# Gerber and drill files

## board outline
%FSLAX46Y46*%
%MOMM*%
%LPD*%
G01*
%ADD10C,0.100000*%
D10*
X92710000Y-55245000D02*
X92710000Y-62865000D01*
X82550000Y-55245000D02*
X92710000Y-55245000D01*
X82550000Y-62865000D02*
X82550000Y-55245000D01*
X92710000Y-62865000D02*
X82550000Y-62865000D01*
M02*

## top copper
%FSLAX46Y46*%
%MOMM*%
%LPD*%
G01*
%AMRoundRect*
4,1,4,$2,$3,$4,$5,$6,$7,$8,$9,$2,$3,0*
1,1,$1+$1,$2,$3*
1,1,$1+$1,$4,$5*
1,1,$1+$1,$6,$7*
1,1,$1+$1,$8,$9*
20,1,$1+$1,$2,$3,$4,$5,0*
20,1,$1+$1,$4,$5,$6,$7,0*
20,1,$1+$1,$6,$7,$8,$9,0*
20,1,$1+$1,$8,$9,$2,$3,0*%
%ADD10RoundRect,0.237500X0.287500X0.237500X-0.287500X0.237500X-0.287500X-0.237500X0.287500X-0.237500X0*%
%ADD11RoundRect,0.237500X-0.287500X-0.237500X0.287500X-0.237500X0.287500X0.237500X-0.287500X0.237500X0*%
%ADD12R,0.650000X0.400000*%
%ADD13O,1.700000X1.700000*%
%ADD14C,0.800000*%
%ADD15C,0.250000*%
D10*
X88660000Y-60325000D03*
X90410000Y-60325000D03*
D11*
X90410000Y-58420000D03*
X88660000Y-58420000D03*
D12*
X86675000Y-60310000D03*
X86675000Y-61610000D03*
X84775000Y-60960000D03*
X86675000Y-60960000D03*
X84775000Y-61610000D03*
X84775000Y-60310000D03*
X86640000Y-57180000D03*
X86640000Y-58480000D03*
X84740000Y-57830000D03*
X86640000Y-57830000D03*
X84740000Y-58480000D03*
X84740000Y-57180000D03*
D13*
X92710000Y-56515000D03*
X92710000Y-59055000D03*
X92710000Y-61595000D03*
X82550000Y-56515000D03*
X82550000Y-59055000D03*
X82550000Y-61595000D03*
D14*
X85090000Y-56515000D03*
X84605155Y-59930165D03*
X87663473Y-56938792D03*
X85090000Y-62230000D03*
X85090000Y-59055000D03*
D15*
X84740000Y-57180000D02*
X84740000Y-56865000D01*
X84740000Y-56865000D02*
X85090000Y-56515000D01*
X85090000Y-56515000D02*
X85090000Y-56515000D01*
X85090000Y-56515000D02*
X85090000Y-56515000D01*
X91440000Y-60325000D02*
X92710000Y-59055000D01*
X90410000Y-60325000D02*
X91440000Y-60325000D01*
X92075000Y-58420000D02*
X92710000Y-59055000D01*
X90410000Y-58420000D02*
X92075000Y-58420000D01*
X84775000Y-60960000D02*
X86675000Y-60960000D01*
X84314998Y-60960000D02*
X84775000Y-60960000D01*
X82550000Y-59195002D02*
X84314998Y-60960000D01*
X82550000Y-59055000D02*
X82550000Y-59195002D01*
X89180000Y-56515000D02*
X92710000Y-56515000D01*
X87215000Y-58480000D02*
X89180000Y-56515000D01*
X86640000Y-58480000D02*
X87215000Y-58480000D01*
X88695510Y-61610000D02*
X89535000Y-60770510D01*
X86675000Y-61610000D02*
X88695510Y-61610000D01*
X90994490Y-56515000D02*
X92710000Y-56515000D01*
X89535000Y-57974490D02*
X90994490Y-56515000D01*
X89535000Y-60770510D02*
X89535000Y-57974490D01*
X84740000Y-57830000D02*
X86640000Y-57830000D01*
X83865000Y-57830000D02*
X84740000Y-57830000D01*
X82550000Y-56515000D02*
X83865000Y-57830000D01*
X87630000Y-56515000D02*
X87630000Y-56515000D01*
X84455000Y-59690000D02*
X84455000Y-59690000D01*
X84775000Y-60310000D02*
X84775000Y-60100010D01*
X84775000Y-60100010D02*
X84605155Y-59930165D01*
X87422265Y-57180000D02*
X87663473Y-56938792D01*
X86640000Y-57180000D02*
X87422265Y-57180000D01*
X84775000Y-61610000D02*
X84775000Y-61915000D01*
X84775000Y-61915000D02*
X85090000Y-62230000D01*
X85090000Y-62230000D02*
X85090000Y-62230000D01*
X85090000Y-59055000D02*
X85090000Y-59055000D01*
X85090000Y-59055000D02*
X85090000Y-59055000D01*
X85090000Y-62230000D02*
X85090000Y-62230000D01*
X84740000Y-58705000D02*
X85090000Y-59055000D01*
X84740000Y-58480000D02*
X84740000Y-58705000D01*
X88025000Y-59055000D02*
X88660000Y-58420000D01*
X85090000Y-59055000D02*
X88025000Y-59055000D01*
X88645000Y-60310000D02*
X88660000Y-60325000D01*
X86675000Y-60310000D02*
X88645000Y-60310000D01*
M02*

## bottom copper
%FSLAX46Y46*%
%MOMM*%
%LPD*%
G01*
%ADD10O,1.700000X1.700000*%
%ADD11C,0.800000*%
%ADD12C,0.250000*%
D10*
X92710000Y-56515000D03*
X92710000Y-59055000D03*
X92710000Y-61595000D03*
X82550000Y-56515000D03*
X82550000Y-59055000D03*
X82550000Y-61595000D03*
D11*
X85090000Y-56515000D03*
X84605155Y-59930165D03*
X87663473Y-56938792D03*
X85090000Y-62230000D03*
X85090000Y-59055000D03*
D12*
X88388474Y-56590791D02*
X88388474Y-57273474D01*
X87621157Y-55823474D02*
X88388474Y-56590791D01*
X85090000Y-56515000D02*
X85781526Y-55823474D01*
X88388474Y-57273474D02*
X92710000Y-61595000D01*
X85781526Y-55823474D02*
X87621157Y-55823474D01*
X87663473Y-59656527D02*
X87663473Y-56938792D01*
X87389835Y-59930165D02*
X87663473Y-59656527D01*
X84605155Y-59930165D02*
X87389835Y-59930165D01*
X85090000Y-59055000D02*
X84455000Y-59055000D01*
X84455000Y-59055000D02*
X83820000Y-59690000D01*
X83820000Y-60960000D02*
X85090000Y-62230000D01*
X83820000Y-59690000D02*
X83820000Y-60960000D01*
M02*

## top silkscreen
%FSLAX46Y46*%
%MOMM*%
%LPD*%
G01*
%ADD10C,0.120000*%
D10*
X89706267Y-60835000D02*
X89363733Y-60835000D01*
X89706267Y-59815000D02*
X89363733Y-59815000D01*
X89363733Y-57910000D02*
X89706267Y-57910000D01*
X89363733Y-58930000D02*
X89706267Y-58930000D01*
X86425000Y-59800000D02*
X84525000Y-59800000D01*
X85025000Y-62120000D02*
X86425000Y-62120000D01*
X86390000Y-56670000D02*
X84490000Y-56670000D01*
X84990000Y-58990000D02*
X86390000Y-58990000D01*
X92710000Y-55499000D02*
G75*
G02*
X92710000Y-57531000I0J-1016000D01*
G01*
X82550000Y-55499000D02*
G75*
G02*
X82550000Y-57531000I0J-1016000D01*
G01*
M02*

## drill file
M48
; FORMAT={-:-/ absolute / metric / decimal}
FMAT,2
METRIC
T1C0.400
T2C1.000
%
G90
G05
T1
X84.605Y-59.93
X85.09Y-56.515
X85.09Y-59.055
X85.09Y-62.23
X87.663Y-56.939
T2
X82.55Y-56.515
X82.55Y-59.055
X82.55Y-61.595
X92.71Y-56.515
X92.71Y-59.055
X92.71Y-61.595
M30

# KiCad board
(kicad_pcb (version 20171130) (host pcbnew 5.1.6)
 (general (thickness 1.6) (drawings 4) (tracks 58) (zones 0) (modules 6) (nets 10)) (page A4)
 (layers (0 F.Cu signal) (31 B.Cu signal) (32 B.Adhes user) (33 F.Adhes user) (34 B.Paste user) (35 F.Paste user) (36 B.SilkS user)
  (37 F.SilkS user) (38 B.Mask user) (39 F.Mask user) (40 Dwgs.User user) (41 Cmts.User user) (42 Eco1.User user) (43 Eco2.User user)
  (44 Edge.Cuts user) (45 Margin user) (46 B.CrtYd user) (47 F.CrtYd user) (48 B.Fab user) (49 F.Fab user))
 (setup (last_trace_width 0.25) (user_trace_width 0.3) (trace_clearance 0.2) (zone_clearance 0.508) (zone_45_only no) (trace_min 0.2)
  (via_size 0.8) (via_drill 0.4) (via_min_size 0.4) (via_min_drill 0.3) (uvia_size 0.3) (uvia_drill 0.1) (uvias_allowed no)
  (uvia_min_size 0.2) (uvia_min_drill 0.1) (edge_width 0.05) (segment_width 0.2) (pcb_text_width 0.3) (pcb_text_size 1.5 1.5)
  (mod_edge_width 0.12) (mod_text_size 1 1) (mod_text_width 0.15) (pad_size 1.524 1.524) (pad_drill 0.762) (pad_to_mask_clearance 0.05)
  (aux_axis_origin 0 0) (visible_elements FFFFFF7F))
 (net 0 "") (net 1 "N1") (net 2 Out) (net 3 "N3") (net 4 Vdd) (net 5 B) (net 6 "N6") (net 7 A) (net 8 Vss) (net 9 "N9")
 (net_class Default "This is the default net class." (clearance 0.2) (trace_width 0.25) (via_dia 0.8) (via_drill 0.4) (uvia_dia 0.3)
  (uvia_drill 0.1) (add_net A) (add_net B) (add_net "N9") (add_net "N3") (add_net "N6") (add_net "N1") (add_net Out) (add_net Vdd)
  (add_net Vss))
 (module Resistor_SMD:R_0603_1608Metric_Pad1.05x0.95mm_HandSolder (layer F.Cu) (at 89.535 60.325 180)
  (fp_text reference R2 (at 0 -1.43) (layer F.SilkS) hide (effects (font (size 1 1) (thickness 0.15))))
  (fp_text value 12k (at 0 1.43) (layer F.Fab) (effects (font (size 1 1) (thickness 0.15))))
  (fp_line (start -0.171267 -0.51) (end 0.171267 -0.51) (layer F.SilkS) (width 0.12))
  (fp_line (start -0.171267 0.51) (end 0.171267 0.51) (layer F.SilkS) (width 0.12))
  (pad 2 smd roundrect (at 0.875 0 180) (size 1.05 0.95) (layers F.Cu F.Paste F.Mask) (roundrect_rratio 0.25) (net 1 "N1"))
  (pad 1 smd roundrect (at -0.875 0 180) (size 1.05 0.95) (layers F.Cu F.Paste F.Mask) (roundrect_rratio 0.25) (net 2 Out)))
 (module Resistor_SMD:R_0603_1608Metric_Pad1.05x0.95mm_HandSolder (layer F.Cu) (at 89.535 58.42)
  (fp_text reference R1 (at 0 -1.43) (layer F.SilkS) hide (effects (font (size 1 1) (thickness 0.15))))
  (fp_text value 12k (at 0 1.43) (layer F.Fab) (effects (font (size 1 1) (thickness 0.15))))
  (fp_line (start -0.171267 -0.51) (end 0.171267 -0.51) (layer F.SilkS) (width 0.12))
  (fp_line (start -0.171267 0.51) (end 0.171267 0.51) (layer F.SilkS) (width 0.12))
  (pad 2 smd roundrect (at 0.875 0) (size 1.05 0.95) (layers F.Cu F.Paste F.Mask) (roundrect_rratio 0.25) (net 2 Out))
  (pad 1 smd roundrect (at -0.875 0) (size 1.05 0.95) (layers F.Cu F.Paste F.Mask) (roundrect_rratio 0.25) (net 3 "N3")))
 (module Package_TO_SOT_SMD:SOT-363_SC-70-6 (layer F.Cu) (at 85.725 60.96)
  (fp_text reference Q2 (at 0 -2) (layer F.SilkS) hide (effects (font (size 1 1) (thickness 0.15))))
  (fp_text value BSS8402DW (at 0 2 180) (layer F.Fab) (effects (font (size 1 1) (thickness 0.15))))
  (fp_line (start 0.7 -1.16) (end -1.2 -1.16) (layer F.SilkS) (width 0.12))
  (fp_line (start -0.7 1.16) (end 0.7 1.16) (layer F.SilkS) (width 0.12))
  (pad 6 smd rect (at 0.95 -0.65) (size 0.65 0.4) (layers F.Cu F.Paste F.Mask) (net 1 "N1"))
  (pad 4 smd rect (at 0.95 0.65) (size 0.65 0.4) (layers F.Cu F.Paste F.Mask) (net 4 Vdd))
  (pad 2 smd rect (at -0.95 0) (size 0.65 0.4) (layers F.Cu F.Paste F.Mask) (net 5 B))
  (pad 5 smd rect (at 0.95 0) (size 0.65 0.4) (layers F.Cu F.Paste F.Mask) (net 5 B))
  (pad 3 smd rect (at -0.95 0.65) (size 0.65 0.4) (layers F.Cu F.Paste F.Mask) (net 3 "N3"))
  (pad 1 smd rect (at -0.95 -0.65) (size 0.65 0.4) (layers F.Cu F.Paste F.Mask) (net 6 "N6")))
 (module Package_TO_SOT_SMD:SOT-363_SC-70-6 (layer F.Cu) (at 85.69 57.83)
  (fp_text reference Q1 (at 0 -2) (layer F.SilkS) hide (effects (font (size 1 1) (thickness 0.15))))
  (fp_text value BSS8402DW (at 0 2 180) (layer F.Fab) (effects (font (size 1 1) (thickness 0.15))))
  (fp_line (start 0.7 -1.16) (end -1.2 -1.16) (layer F.SilkS) (width 0.12))
  (fp_line (start -0.7 1.16) (end 0.7 1.16) (layer F.SilkS) (width 0.12))
  (pad 6 smd rect (at 0.95 -0.65) (size 0.65 0.4) (layers F.Cu F.Paste F.Mask) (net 6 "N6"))
  (pad 4 smd rect (at 0.95 0.65) (size 0.65 0.4) (layers F.Cu F.Paste F.Mask) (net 4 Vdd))
  (pad 2 smd rect (at -0.95 0) (size 0.65 0.4) (layers F.Cu F.Paste F.Mask) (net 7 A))
  (pad 5 smd rect (at 0.95 0) (size 0.65 0.4) (layers F.Cu F.Paste F.Mask) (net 7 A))
  (pad 3 smd rect (at -0.95 0.65) (size 0.65 0.4) (layers F.Cu F.Paste F.Mask) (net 3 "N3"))
  (pad 1 smd rect (at -0.95 -0.65) (size 0.65 0.4) (layers F.Cu F.Paste F.Mask) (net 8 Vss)))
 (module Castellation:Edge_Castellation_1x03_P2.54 (layer F.Cu) (at 92.71 56.515)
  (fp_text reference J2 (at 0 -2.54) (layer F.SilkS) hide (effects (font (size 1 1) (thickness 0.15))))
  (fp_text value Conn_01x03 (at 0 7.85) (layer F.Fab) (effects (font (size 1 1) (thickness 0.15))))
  (fp_arc (start 0 0) (end 0 1.016) (angle -180) (layer F.SilkS) (width 0.12))
  (pad 1 thru_hole oval (at 0 0) (size 1.7 1.7) (drill 1) (layers *.Cu *.Mask) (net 4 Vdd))
  (pad 2 thru_hole oval (at 0 2.54) (size 1.7 1.7) (drill 1) (layers *.Cu *.Mask) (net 2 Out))
  (pad 3 thru_hole oval (at 0 5.08) (size 1.7 1.7) (drill 1) (layers *.Cu *.Mask) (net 8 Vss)))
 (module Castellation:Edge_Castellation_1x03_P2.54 (layer F.Cu) (at 82.55 56.515)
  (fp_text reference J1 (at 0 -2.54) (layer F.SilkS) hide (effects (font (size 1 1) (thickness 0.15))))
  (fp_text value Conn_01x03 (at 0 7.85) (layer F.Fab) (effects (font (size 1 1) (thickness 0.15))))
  (fp_arc (start 0 0) (end 0 1.016) (angle -180) (layer F.SilkS) (width 0.12))
  (pad 1 thru_hole oval (at 0 0) (size 1.7 1.7) (drill 1) (layers *.Cu *.Mask) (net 7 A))
  (pad 2 thru_hole oval (at 0 2.54) (size 1.7 1.7) (drill 1) (layers *.Cu *.Mask) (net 5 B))
  (pad 3 thru_hole oval (at 0 5.08) (size 1.7 1.7) (drill 1) (layers *.Cu *.Mask) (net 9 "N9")))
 (gr_line (start 92.71 55.245) (end 92.71 62.865) (layer Edge.Cuts) (width 0.1))
 (gr_line (start 82.55 55.245) (end 92.71 55.245) (layer Edge.Cuts) (width 0.1))
 (gr_line (start 82.55 62.865) (end 82.55 55.245) (layer Edge.Cuts) (width 0.1))
 (gr_line (start 92.71 62.865) (end 82.55 62.865) (layer Edge.Cuts) (width 0.1))
 (segment (start 84.74 57.18) (end 84.74 56.865) (width 0.25) (layer F.Cu) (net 8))
 (segment (start 84.74 56.865) (end 85.09 56.515) (width 0.25) (layer F.Cu) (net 8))
 (segment (start 85.09 56.515) (end 85.09 56.515) (width 0.25) (layer F.Cu) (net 8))
 (segment (start 85.09 56.515) (end 85.09 56.515) (width 0.25) (layer F.Cu) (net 8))
 (via (at 85.09 56.515) (size 0.8) (drill 0.4) (layers F.Cu B.Cu) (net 8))
 (segment (start 88.388474 56.590791) (end 88.388474 57.273474) (width 0.25) (layer B.Cu) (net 8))
 (segment (start 87.621157 55.823474) (end 88.388474 56.590791) (width 0.25) (layer B.Cu) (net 8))
 (segment (start 85.09 56.515) (end 85.781526 55.823474) (width 0.25) (layer B.Cu) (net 8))
 (segment (start 88.388474 57.273474) (end 92.71 61.595) (width 0.25) (layer B.Cu) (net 8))
 (segment (start 85.781526 55.823474) (end 87.621157 55.823474) (width 0.25) (layer B.Cu) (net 8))
 (segment (start 91.44 60.325) (end 92.71 59.055) (width 0.25) (layer F.Cu) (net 2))
 (segment (start 90.41 60.325) (end 91.44 60.325) (width 0.25) (layer F.Cu) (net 2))
 (segment (start 92.075 58.42) (end 92.71 59.055) (width 0.25) (layer F.Cu) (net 2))
 (segment (start 90.41 58.42) (end 92.075 58.42) (width 0.25) (layer F.Cu) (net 2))
 (segment (start 84.775 60.96) (end 86.675 60.96) (width 0.25) (layer F.Cu) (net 5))
 (segment (start 84.314998 60.96) (end 84.775 60.96) (width 0.25) (layer F.Cu) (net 5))
 (segment (start 82.55 59.195002) (end 84.314998 60.96) (width 0.25) (layer F.Cu) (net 5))
 (segment (start 82.55 59.055) (end 82.55 59.195002) (width 0.25) (layer F.Cu) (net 5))
 (segment (start 89.18 56.515) (end 92.71 56.515) (width 0.25) (layer F.Cu) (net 4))
 (segment (start 87.215 58.48) (end 89.18 56.515) (width 0.25) (layer F.Cu) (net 4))
 (segment (start 86.64 58.48) (end 87.215 58.48) (width 0.25) (layer F.Cu) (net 4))
 (segment (start 88.69551 61.61) (end 89.535 60.77051) (width 0.25) (layer F.Cu) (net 4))
 (segment (start 86.675 61.61) (end 88.69551 61.61) (width 0.25) (layer F.Cu) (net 4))
 (segment (start 90.99449 56.515) (end 92.71 56.515) (width 0.25) (layer F.Cu) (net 4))
 (segment (start 89.535 57.97449) (end 90.99449 56.515) (width 0.25) (layer F.Cu) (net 4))
 (segment (start 89.535 60.77051) (end 89.535 57.97449) (width 0.25) (layer F.Cu) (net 4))
 (segment (start 84.74 57.83) (end 86.64 57.83) (width 0.25) (layer F.Cu) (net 7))
 (segment (start 83.865 57.83) (end 84.74 57.83) (width 0.25) (layer F.Cu) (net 7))
 (segment (start 82.55 56.515) (end 83.865 57.83) (width 0.25) (layer F.Cu) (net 7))
 (segment (start 87.63 56.515) (end 87.63 56.515) (width 0.25) (layer F.Cu) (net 6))
 (segment (start 84.455 59.69) (end 84.455 59.69) (width 0.25) (layer F.Cu) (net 6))
 (segment (start 84.775 60.31) (end 84.775 60.10001) (width 0.25) (layer F.Cu) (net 6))
 (segment (start 84.775 60.10001) (end 84.605155 59.930165) (width 0.25) (layer F.Cu) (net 6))
 (via (at 84.605155 59.930165) (size 0.8) (drill 0.4) (layers F.Cu B.Cu) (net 6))
 (segment (start 87.663473 59.656527) (end 87.663473 56.938792) (width 0.25) (layer B.Cu) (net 6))
 (segment (start 87.422265 57.18) (end 87.663473 56.938792) (width 0.25) (layer F.Cu) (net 6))
 (via (at 87.663473 56.938792) (size 0.8) (drill 0.4) (layers F.Cu B.Cu) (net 6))
 (segment (start 86.64 57.18) (end 87.422265 57.18) (width 0.25) (layer F.Cu) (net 6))
 (segment (start 87.389835 59.930165) (end 87.663473 59.656527) (width 0.25) (layer B.Cu) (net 6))
 (segment (start 84.605155 59.930165) (end 87.389835 59.930165) (width 0.25) (layer B.Cu) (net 6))
 (segment (start 84.775 61.61) (end 84.775 61.915) (width 0.25) (layer F.Cu) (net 3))
 (segment (start 84.775 61.915) (end 85.09 62.23) (width 0.25) (layer F.Cu) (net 3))
 (segment (start 85.09 62.23) (end 85.09 62.23) (width 0.25) (layer F.Cu) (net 3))
 (segment (start 85.09 59.055) (end 85.09 59.055) (width 0.25) (layer F.Cu) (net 3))
 (segment (start 85.09 59.055) (end 85.09 59.055) (width 0.25) (layer F.Cu) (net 3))
 (segment (start 85.09 62.23) (end 85.09 62.23) (width 0.25) (layer F.Cu) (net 3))
 (via (at 85.09 62.23) (size 0.8) (drill 0.4) (layers F.Cu B.Cu) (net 3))
 (segment (start 84.74 58.705) (end 85.09 59.055) (width 0.25) (layer F.Cu) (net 3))
 (segment (start 84.74 58.48) (end 84.74 58.705) (width 0.25) (layer F.Cu) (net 3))
 (segment (start 88.025 59.055) (end 88.66 58.42) (width 0.25) (layer F.Cu) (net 3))
 (via (at 85.09 59.055) (size 0.8) (drill 0.4) (layers F.Cu B.Cu) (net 3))
 (segment (start 85.09 59.055) (end 88.025 59.055) (width 0.25) (layer F.Cu) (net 3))
 (segment (start 85.09 59.055) (end 84.455 59.055) (width 0.25) (layer B.Cu) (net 3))
 (segment (start 84.455 59.055) (end 83.82 59.69) (width 0.25) (layer B.Cu) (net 3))
 (segment (start 83.82 60.96) (end 85.09 62.23) (width 0.25) (layer B.Cu) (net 3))
 (segment (start 83.82 59.69) (end 83.82 60.96) (width 0.25) (layer B.Cu) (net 3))
 (segment (start 88.645 60.31) (end 88.66 60.325) (width 0.25) (layer F.Cu) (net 1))
 (segment (start 86.675 60.31) (end 88.645 60.31) (width 0.25) (layer F.Cu) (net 1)))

